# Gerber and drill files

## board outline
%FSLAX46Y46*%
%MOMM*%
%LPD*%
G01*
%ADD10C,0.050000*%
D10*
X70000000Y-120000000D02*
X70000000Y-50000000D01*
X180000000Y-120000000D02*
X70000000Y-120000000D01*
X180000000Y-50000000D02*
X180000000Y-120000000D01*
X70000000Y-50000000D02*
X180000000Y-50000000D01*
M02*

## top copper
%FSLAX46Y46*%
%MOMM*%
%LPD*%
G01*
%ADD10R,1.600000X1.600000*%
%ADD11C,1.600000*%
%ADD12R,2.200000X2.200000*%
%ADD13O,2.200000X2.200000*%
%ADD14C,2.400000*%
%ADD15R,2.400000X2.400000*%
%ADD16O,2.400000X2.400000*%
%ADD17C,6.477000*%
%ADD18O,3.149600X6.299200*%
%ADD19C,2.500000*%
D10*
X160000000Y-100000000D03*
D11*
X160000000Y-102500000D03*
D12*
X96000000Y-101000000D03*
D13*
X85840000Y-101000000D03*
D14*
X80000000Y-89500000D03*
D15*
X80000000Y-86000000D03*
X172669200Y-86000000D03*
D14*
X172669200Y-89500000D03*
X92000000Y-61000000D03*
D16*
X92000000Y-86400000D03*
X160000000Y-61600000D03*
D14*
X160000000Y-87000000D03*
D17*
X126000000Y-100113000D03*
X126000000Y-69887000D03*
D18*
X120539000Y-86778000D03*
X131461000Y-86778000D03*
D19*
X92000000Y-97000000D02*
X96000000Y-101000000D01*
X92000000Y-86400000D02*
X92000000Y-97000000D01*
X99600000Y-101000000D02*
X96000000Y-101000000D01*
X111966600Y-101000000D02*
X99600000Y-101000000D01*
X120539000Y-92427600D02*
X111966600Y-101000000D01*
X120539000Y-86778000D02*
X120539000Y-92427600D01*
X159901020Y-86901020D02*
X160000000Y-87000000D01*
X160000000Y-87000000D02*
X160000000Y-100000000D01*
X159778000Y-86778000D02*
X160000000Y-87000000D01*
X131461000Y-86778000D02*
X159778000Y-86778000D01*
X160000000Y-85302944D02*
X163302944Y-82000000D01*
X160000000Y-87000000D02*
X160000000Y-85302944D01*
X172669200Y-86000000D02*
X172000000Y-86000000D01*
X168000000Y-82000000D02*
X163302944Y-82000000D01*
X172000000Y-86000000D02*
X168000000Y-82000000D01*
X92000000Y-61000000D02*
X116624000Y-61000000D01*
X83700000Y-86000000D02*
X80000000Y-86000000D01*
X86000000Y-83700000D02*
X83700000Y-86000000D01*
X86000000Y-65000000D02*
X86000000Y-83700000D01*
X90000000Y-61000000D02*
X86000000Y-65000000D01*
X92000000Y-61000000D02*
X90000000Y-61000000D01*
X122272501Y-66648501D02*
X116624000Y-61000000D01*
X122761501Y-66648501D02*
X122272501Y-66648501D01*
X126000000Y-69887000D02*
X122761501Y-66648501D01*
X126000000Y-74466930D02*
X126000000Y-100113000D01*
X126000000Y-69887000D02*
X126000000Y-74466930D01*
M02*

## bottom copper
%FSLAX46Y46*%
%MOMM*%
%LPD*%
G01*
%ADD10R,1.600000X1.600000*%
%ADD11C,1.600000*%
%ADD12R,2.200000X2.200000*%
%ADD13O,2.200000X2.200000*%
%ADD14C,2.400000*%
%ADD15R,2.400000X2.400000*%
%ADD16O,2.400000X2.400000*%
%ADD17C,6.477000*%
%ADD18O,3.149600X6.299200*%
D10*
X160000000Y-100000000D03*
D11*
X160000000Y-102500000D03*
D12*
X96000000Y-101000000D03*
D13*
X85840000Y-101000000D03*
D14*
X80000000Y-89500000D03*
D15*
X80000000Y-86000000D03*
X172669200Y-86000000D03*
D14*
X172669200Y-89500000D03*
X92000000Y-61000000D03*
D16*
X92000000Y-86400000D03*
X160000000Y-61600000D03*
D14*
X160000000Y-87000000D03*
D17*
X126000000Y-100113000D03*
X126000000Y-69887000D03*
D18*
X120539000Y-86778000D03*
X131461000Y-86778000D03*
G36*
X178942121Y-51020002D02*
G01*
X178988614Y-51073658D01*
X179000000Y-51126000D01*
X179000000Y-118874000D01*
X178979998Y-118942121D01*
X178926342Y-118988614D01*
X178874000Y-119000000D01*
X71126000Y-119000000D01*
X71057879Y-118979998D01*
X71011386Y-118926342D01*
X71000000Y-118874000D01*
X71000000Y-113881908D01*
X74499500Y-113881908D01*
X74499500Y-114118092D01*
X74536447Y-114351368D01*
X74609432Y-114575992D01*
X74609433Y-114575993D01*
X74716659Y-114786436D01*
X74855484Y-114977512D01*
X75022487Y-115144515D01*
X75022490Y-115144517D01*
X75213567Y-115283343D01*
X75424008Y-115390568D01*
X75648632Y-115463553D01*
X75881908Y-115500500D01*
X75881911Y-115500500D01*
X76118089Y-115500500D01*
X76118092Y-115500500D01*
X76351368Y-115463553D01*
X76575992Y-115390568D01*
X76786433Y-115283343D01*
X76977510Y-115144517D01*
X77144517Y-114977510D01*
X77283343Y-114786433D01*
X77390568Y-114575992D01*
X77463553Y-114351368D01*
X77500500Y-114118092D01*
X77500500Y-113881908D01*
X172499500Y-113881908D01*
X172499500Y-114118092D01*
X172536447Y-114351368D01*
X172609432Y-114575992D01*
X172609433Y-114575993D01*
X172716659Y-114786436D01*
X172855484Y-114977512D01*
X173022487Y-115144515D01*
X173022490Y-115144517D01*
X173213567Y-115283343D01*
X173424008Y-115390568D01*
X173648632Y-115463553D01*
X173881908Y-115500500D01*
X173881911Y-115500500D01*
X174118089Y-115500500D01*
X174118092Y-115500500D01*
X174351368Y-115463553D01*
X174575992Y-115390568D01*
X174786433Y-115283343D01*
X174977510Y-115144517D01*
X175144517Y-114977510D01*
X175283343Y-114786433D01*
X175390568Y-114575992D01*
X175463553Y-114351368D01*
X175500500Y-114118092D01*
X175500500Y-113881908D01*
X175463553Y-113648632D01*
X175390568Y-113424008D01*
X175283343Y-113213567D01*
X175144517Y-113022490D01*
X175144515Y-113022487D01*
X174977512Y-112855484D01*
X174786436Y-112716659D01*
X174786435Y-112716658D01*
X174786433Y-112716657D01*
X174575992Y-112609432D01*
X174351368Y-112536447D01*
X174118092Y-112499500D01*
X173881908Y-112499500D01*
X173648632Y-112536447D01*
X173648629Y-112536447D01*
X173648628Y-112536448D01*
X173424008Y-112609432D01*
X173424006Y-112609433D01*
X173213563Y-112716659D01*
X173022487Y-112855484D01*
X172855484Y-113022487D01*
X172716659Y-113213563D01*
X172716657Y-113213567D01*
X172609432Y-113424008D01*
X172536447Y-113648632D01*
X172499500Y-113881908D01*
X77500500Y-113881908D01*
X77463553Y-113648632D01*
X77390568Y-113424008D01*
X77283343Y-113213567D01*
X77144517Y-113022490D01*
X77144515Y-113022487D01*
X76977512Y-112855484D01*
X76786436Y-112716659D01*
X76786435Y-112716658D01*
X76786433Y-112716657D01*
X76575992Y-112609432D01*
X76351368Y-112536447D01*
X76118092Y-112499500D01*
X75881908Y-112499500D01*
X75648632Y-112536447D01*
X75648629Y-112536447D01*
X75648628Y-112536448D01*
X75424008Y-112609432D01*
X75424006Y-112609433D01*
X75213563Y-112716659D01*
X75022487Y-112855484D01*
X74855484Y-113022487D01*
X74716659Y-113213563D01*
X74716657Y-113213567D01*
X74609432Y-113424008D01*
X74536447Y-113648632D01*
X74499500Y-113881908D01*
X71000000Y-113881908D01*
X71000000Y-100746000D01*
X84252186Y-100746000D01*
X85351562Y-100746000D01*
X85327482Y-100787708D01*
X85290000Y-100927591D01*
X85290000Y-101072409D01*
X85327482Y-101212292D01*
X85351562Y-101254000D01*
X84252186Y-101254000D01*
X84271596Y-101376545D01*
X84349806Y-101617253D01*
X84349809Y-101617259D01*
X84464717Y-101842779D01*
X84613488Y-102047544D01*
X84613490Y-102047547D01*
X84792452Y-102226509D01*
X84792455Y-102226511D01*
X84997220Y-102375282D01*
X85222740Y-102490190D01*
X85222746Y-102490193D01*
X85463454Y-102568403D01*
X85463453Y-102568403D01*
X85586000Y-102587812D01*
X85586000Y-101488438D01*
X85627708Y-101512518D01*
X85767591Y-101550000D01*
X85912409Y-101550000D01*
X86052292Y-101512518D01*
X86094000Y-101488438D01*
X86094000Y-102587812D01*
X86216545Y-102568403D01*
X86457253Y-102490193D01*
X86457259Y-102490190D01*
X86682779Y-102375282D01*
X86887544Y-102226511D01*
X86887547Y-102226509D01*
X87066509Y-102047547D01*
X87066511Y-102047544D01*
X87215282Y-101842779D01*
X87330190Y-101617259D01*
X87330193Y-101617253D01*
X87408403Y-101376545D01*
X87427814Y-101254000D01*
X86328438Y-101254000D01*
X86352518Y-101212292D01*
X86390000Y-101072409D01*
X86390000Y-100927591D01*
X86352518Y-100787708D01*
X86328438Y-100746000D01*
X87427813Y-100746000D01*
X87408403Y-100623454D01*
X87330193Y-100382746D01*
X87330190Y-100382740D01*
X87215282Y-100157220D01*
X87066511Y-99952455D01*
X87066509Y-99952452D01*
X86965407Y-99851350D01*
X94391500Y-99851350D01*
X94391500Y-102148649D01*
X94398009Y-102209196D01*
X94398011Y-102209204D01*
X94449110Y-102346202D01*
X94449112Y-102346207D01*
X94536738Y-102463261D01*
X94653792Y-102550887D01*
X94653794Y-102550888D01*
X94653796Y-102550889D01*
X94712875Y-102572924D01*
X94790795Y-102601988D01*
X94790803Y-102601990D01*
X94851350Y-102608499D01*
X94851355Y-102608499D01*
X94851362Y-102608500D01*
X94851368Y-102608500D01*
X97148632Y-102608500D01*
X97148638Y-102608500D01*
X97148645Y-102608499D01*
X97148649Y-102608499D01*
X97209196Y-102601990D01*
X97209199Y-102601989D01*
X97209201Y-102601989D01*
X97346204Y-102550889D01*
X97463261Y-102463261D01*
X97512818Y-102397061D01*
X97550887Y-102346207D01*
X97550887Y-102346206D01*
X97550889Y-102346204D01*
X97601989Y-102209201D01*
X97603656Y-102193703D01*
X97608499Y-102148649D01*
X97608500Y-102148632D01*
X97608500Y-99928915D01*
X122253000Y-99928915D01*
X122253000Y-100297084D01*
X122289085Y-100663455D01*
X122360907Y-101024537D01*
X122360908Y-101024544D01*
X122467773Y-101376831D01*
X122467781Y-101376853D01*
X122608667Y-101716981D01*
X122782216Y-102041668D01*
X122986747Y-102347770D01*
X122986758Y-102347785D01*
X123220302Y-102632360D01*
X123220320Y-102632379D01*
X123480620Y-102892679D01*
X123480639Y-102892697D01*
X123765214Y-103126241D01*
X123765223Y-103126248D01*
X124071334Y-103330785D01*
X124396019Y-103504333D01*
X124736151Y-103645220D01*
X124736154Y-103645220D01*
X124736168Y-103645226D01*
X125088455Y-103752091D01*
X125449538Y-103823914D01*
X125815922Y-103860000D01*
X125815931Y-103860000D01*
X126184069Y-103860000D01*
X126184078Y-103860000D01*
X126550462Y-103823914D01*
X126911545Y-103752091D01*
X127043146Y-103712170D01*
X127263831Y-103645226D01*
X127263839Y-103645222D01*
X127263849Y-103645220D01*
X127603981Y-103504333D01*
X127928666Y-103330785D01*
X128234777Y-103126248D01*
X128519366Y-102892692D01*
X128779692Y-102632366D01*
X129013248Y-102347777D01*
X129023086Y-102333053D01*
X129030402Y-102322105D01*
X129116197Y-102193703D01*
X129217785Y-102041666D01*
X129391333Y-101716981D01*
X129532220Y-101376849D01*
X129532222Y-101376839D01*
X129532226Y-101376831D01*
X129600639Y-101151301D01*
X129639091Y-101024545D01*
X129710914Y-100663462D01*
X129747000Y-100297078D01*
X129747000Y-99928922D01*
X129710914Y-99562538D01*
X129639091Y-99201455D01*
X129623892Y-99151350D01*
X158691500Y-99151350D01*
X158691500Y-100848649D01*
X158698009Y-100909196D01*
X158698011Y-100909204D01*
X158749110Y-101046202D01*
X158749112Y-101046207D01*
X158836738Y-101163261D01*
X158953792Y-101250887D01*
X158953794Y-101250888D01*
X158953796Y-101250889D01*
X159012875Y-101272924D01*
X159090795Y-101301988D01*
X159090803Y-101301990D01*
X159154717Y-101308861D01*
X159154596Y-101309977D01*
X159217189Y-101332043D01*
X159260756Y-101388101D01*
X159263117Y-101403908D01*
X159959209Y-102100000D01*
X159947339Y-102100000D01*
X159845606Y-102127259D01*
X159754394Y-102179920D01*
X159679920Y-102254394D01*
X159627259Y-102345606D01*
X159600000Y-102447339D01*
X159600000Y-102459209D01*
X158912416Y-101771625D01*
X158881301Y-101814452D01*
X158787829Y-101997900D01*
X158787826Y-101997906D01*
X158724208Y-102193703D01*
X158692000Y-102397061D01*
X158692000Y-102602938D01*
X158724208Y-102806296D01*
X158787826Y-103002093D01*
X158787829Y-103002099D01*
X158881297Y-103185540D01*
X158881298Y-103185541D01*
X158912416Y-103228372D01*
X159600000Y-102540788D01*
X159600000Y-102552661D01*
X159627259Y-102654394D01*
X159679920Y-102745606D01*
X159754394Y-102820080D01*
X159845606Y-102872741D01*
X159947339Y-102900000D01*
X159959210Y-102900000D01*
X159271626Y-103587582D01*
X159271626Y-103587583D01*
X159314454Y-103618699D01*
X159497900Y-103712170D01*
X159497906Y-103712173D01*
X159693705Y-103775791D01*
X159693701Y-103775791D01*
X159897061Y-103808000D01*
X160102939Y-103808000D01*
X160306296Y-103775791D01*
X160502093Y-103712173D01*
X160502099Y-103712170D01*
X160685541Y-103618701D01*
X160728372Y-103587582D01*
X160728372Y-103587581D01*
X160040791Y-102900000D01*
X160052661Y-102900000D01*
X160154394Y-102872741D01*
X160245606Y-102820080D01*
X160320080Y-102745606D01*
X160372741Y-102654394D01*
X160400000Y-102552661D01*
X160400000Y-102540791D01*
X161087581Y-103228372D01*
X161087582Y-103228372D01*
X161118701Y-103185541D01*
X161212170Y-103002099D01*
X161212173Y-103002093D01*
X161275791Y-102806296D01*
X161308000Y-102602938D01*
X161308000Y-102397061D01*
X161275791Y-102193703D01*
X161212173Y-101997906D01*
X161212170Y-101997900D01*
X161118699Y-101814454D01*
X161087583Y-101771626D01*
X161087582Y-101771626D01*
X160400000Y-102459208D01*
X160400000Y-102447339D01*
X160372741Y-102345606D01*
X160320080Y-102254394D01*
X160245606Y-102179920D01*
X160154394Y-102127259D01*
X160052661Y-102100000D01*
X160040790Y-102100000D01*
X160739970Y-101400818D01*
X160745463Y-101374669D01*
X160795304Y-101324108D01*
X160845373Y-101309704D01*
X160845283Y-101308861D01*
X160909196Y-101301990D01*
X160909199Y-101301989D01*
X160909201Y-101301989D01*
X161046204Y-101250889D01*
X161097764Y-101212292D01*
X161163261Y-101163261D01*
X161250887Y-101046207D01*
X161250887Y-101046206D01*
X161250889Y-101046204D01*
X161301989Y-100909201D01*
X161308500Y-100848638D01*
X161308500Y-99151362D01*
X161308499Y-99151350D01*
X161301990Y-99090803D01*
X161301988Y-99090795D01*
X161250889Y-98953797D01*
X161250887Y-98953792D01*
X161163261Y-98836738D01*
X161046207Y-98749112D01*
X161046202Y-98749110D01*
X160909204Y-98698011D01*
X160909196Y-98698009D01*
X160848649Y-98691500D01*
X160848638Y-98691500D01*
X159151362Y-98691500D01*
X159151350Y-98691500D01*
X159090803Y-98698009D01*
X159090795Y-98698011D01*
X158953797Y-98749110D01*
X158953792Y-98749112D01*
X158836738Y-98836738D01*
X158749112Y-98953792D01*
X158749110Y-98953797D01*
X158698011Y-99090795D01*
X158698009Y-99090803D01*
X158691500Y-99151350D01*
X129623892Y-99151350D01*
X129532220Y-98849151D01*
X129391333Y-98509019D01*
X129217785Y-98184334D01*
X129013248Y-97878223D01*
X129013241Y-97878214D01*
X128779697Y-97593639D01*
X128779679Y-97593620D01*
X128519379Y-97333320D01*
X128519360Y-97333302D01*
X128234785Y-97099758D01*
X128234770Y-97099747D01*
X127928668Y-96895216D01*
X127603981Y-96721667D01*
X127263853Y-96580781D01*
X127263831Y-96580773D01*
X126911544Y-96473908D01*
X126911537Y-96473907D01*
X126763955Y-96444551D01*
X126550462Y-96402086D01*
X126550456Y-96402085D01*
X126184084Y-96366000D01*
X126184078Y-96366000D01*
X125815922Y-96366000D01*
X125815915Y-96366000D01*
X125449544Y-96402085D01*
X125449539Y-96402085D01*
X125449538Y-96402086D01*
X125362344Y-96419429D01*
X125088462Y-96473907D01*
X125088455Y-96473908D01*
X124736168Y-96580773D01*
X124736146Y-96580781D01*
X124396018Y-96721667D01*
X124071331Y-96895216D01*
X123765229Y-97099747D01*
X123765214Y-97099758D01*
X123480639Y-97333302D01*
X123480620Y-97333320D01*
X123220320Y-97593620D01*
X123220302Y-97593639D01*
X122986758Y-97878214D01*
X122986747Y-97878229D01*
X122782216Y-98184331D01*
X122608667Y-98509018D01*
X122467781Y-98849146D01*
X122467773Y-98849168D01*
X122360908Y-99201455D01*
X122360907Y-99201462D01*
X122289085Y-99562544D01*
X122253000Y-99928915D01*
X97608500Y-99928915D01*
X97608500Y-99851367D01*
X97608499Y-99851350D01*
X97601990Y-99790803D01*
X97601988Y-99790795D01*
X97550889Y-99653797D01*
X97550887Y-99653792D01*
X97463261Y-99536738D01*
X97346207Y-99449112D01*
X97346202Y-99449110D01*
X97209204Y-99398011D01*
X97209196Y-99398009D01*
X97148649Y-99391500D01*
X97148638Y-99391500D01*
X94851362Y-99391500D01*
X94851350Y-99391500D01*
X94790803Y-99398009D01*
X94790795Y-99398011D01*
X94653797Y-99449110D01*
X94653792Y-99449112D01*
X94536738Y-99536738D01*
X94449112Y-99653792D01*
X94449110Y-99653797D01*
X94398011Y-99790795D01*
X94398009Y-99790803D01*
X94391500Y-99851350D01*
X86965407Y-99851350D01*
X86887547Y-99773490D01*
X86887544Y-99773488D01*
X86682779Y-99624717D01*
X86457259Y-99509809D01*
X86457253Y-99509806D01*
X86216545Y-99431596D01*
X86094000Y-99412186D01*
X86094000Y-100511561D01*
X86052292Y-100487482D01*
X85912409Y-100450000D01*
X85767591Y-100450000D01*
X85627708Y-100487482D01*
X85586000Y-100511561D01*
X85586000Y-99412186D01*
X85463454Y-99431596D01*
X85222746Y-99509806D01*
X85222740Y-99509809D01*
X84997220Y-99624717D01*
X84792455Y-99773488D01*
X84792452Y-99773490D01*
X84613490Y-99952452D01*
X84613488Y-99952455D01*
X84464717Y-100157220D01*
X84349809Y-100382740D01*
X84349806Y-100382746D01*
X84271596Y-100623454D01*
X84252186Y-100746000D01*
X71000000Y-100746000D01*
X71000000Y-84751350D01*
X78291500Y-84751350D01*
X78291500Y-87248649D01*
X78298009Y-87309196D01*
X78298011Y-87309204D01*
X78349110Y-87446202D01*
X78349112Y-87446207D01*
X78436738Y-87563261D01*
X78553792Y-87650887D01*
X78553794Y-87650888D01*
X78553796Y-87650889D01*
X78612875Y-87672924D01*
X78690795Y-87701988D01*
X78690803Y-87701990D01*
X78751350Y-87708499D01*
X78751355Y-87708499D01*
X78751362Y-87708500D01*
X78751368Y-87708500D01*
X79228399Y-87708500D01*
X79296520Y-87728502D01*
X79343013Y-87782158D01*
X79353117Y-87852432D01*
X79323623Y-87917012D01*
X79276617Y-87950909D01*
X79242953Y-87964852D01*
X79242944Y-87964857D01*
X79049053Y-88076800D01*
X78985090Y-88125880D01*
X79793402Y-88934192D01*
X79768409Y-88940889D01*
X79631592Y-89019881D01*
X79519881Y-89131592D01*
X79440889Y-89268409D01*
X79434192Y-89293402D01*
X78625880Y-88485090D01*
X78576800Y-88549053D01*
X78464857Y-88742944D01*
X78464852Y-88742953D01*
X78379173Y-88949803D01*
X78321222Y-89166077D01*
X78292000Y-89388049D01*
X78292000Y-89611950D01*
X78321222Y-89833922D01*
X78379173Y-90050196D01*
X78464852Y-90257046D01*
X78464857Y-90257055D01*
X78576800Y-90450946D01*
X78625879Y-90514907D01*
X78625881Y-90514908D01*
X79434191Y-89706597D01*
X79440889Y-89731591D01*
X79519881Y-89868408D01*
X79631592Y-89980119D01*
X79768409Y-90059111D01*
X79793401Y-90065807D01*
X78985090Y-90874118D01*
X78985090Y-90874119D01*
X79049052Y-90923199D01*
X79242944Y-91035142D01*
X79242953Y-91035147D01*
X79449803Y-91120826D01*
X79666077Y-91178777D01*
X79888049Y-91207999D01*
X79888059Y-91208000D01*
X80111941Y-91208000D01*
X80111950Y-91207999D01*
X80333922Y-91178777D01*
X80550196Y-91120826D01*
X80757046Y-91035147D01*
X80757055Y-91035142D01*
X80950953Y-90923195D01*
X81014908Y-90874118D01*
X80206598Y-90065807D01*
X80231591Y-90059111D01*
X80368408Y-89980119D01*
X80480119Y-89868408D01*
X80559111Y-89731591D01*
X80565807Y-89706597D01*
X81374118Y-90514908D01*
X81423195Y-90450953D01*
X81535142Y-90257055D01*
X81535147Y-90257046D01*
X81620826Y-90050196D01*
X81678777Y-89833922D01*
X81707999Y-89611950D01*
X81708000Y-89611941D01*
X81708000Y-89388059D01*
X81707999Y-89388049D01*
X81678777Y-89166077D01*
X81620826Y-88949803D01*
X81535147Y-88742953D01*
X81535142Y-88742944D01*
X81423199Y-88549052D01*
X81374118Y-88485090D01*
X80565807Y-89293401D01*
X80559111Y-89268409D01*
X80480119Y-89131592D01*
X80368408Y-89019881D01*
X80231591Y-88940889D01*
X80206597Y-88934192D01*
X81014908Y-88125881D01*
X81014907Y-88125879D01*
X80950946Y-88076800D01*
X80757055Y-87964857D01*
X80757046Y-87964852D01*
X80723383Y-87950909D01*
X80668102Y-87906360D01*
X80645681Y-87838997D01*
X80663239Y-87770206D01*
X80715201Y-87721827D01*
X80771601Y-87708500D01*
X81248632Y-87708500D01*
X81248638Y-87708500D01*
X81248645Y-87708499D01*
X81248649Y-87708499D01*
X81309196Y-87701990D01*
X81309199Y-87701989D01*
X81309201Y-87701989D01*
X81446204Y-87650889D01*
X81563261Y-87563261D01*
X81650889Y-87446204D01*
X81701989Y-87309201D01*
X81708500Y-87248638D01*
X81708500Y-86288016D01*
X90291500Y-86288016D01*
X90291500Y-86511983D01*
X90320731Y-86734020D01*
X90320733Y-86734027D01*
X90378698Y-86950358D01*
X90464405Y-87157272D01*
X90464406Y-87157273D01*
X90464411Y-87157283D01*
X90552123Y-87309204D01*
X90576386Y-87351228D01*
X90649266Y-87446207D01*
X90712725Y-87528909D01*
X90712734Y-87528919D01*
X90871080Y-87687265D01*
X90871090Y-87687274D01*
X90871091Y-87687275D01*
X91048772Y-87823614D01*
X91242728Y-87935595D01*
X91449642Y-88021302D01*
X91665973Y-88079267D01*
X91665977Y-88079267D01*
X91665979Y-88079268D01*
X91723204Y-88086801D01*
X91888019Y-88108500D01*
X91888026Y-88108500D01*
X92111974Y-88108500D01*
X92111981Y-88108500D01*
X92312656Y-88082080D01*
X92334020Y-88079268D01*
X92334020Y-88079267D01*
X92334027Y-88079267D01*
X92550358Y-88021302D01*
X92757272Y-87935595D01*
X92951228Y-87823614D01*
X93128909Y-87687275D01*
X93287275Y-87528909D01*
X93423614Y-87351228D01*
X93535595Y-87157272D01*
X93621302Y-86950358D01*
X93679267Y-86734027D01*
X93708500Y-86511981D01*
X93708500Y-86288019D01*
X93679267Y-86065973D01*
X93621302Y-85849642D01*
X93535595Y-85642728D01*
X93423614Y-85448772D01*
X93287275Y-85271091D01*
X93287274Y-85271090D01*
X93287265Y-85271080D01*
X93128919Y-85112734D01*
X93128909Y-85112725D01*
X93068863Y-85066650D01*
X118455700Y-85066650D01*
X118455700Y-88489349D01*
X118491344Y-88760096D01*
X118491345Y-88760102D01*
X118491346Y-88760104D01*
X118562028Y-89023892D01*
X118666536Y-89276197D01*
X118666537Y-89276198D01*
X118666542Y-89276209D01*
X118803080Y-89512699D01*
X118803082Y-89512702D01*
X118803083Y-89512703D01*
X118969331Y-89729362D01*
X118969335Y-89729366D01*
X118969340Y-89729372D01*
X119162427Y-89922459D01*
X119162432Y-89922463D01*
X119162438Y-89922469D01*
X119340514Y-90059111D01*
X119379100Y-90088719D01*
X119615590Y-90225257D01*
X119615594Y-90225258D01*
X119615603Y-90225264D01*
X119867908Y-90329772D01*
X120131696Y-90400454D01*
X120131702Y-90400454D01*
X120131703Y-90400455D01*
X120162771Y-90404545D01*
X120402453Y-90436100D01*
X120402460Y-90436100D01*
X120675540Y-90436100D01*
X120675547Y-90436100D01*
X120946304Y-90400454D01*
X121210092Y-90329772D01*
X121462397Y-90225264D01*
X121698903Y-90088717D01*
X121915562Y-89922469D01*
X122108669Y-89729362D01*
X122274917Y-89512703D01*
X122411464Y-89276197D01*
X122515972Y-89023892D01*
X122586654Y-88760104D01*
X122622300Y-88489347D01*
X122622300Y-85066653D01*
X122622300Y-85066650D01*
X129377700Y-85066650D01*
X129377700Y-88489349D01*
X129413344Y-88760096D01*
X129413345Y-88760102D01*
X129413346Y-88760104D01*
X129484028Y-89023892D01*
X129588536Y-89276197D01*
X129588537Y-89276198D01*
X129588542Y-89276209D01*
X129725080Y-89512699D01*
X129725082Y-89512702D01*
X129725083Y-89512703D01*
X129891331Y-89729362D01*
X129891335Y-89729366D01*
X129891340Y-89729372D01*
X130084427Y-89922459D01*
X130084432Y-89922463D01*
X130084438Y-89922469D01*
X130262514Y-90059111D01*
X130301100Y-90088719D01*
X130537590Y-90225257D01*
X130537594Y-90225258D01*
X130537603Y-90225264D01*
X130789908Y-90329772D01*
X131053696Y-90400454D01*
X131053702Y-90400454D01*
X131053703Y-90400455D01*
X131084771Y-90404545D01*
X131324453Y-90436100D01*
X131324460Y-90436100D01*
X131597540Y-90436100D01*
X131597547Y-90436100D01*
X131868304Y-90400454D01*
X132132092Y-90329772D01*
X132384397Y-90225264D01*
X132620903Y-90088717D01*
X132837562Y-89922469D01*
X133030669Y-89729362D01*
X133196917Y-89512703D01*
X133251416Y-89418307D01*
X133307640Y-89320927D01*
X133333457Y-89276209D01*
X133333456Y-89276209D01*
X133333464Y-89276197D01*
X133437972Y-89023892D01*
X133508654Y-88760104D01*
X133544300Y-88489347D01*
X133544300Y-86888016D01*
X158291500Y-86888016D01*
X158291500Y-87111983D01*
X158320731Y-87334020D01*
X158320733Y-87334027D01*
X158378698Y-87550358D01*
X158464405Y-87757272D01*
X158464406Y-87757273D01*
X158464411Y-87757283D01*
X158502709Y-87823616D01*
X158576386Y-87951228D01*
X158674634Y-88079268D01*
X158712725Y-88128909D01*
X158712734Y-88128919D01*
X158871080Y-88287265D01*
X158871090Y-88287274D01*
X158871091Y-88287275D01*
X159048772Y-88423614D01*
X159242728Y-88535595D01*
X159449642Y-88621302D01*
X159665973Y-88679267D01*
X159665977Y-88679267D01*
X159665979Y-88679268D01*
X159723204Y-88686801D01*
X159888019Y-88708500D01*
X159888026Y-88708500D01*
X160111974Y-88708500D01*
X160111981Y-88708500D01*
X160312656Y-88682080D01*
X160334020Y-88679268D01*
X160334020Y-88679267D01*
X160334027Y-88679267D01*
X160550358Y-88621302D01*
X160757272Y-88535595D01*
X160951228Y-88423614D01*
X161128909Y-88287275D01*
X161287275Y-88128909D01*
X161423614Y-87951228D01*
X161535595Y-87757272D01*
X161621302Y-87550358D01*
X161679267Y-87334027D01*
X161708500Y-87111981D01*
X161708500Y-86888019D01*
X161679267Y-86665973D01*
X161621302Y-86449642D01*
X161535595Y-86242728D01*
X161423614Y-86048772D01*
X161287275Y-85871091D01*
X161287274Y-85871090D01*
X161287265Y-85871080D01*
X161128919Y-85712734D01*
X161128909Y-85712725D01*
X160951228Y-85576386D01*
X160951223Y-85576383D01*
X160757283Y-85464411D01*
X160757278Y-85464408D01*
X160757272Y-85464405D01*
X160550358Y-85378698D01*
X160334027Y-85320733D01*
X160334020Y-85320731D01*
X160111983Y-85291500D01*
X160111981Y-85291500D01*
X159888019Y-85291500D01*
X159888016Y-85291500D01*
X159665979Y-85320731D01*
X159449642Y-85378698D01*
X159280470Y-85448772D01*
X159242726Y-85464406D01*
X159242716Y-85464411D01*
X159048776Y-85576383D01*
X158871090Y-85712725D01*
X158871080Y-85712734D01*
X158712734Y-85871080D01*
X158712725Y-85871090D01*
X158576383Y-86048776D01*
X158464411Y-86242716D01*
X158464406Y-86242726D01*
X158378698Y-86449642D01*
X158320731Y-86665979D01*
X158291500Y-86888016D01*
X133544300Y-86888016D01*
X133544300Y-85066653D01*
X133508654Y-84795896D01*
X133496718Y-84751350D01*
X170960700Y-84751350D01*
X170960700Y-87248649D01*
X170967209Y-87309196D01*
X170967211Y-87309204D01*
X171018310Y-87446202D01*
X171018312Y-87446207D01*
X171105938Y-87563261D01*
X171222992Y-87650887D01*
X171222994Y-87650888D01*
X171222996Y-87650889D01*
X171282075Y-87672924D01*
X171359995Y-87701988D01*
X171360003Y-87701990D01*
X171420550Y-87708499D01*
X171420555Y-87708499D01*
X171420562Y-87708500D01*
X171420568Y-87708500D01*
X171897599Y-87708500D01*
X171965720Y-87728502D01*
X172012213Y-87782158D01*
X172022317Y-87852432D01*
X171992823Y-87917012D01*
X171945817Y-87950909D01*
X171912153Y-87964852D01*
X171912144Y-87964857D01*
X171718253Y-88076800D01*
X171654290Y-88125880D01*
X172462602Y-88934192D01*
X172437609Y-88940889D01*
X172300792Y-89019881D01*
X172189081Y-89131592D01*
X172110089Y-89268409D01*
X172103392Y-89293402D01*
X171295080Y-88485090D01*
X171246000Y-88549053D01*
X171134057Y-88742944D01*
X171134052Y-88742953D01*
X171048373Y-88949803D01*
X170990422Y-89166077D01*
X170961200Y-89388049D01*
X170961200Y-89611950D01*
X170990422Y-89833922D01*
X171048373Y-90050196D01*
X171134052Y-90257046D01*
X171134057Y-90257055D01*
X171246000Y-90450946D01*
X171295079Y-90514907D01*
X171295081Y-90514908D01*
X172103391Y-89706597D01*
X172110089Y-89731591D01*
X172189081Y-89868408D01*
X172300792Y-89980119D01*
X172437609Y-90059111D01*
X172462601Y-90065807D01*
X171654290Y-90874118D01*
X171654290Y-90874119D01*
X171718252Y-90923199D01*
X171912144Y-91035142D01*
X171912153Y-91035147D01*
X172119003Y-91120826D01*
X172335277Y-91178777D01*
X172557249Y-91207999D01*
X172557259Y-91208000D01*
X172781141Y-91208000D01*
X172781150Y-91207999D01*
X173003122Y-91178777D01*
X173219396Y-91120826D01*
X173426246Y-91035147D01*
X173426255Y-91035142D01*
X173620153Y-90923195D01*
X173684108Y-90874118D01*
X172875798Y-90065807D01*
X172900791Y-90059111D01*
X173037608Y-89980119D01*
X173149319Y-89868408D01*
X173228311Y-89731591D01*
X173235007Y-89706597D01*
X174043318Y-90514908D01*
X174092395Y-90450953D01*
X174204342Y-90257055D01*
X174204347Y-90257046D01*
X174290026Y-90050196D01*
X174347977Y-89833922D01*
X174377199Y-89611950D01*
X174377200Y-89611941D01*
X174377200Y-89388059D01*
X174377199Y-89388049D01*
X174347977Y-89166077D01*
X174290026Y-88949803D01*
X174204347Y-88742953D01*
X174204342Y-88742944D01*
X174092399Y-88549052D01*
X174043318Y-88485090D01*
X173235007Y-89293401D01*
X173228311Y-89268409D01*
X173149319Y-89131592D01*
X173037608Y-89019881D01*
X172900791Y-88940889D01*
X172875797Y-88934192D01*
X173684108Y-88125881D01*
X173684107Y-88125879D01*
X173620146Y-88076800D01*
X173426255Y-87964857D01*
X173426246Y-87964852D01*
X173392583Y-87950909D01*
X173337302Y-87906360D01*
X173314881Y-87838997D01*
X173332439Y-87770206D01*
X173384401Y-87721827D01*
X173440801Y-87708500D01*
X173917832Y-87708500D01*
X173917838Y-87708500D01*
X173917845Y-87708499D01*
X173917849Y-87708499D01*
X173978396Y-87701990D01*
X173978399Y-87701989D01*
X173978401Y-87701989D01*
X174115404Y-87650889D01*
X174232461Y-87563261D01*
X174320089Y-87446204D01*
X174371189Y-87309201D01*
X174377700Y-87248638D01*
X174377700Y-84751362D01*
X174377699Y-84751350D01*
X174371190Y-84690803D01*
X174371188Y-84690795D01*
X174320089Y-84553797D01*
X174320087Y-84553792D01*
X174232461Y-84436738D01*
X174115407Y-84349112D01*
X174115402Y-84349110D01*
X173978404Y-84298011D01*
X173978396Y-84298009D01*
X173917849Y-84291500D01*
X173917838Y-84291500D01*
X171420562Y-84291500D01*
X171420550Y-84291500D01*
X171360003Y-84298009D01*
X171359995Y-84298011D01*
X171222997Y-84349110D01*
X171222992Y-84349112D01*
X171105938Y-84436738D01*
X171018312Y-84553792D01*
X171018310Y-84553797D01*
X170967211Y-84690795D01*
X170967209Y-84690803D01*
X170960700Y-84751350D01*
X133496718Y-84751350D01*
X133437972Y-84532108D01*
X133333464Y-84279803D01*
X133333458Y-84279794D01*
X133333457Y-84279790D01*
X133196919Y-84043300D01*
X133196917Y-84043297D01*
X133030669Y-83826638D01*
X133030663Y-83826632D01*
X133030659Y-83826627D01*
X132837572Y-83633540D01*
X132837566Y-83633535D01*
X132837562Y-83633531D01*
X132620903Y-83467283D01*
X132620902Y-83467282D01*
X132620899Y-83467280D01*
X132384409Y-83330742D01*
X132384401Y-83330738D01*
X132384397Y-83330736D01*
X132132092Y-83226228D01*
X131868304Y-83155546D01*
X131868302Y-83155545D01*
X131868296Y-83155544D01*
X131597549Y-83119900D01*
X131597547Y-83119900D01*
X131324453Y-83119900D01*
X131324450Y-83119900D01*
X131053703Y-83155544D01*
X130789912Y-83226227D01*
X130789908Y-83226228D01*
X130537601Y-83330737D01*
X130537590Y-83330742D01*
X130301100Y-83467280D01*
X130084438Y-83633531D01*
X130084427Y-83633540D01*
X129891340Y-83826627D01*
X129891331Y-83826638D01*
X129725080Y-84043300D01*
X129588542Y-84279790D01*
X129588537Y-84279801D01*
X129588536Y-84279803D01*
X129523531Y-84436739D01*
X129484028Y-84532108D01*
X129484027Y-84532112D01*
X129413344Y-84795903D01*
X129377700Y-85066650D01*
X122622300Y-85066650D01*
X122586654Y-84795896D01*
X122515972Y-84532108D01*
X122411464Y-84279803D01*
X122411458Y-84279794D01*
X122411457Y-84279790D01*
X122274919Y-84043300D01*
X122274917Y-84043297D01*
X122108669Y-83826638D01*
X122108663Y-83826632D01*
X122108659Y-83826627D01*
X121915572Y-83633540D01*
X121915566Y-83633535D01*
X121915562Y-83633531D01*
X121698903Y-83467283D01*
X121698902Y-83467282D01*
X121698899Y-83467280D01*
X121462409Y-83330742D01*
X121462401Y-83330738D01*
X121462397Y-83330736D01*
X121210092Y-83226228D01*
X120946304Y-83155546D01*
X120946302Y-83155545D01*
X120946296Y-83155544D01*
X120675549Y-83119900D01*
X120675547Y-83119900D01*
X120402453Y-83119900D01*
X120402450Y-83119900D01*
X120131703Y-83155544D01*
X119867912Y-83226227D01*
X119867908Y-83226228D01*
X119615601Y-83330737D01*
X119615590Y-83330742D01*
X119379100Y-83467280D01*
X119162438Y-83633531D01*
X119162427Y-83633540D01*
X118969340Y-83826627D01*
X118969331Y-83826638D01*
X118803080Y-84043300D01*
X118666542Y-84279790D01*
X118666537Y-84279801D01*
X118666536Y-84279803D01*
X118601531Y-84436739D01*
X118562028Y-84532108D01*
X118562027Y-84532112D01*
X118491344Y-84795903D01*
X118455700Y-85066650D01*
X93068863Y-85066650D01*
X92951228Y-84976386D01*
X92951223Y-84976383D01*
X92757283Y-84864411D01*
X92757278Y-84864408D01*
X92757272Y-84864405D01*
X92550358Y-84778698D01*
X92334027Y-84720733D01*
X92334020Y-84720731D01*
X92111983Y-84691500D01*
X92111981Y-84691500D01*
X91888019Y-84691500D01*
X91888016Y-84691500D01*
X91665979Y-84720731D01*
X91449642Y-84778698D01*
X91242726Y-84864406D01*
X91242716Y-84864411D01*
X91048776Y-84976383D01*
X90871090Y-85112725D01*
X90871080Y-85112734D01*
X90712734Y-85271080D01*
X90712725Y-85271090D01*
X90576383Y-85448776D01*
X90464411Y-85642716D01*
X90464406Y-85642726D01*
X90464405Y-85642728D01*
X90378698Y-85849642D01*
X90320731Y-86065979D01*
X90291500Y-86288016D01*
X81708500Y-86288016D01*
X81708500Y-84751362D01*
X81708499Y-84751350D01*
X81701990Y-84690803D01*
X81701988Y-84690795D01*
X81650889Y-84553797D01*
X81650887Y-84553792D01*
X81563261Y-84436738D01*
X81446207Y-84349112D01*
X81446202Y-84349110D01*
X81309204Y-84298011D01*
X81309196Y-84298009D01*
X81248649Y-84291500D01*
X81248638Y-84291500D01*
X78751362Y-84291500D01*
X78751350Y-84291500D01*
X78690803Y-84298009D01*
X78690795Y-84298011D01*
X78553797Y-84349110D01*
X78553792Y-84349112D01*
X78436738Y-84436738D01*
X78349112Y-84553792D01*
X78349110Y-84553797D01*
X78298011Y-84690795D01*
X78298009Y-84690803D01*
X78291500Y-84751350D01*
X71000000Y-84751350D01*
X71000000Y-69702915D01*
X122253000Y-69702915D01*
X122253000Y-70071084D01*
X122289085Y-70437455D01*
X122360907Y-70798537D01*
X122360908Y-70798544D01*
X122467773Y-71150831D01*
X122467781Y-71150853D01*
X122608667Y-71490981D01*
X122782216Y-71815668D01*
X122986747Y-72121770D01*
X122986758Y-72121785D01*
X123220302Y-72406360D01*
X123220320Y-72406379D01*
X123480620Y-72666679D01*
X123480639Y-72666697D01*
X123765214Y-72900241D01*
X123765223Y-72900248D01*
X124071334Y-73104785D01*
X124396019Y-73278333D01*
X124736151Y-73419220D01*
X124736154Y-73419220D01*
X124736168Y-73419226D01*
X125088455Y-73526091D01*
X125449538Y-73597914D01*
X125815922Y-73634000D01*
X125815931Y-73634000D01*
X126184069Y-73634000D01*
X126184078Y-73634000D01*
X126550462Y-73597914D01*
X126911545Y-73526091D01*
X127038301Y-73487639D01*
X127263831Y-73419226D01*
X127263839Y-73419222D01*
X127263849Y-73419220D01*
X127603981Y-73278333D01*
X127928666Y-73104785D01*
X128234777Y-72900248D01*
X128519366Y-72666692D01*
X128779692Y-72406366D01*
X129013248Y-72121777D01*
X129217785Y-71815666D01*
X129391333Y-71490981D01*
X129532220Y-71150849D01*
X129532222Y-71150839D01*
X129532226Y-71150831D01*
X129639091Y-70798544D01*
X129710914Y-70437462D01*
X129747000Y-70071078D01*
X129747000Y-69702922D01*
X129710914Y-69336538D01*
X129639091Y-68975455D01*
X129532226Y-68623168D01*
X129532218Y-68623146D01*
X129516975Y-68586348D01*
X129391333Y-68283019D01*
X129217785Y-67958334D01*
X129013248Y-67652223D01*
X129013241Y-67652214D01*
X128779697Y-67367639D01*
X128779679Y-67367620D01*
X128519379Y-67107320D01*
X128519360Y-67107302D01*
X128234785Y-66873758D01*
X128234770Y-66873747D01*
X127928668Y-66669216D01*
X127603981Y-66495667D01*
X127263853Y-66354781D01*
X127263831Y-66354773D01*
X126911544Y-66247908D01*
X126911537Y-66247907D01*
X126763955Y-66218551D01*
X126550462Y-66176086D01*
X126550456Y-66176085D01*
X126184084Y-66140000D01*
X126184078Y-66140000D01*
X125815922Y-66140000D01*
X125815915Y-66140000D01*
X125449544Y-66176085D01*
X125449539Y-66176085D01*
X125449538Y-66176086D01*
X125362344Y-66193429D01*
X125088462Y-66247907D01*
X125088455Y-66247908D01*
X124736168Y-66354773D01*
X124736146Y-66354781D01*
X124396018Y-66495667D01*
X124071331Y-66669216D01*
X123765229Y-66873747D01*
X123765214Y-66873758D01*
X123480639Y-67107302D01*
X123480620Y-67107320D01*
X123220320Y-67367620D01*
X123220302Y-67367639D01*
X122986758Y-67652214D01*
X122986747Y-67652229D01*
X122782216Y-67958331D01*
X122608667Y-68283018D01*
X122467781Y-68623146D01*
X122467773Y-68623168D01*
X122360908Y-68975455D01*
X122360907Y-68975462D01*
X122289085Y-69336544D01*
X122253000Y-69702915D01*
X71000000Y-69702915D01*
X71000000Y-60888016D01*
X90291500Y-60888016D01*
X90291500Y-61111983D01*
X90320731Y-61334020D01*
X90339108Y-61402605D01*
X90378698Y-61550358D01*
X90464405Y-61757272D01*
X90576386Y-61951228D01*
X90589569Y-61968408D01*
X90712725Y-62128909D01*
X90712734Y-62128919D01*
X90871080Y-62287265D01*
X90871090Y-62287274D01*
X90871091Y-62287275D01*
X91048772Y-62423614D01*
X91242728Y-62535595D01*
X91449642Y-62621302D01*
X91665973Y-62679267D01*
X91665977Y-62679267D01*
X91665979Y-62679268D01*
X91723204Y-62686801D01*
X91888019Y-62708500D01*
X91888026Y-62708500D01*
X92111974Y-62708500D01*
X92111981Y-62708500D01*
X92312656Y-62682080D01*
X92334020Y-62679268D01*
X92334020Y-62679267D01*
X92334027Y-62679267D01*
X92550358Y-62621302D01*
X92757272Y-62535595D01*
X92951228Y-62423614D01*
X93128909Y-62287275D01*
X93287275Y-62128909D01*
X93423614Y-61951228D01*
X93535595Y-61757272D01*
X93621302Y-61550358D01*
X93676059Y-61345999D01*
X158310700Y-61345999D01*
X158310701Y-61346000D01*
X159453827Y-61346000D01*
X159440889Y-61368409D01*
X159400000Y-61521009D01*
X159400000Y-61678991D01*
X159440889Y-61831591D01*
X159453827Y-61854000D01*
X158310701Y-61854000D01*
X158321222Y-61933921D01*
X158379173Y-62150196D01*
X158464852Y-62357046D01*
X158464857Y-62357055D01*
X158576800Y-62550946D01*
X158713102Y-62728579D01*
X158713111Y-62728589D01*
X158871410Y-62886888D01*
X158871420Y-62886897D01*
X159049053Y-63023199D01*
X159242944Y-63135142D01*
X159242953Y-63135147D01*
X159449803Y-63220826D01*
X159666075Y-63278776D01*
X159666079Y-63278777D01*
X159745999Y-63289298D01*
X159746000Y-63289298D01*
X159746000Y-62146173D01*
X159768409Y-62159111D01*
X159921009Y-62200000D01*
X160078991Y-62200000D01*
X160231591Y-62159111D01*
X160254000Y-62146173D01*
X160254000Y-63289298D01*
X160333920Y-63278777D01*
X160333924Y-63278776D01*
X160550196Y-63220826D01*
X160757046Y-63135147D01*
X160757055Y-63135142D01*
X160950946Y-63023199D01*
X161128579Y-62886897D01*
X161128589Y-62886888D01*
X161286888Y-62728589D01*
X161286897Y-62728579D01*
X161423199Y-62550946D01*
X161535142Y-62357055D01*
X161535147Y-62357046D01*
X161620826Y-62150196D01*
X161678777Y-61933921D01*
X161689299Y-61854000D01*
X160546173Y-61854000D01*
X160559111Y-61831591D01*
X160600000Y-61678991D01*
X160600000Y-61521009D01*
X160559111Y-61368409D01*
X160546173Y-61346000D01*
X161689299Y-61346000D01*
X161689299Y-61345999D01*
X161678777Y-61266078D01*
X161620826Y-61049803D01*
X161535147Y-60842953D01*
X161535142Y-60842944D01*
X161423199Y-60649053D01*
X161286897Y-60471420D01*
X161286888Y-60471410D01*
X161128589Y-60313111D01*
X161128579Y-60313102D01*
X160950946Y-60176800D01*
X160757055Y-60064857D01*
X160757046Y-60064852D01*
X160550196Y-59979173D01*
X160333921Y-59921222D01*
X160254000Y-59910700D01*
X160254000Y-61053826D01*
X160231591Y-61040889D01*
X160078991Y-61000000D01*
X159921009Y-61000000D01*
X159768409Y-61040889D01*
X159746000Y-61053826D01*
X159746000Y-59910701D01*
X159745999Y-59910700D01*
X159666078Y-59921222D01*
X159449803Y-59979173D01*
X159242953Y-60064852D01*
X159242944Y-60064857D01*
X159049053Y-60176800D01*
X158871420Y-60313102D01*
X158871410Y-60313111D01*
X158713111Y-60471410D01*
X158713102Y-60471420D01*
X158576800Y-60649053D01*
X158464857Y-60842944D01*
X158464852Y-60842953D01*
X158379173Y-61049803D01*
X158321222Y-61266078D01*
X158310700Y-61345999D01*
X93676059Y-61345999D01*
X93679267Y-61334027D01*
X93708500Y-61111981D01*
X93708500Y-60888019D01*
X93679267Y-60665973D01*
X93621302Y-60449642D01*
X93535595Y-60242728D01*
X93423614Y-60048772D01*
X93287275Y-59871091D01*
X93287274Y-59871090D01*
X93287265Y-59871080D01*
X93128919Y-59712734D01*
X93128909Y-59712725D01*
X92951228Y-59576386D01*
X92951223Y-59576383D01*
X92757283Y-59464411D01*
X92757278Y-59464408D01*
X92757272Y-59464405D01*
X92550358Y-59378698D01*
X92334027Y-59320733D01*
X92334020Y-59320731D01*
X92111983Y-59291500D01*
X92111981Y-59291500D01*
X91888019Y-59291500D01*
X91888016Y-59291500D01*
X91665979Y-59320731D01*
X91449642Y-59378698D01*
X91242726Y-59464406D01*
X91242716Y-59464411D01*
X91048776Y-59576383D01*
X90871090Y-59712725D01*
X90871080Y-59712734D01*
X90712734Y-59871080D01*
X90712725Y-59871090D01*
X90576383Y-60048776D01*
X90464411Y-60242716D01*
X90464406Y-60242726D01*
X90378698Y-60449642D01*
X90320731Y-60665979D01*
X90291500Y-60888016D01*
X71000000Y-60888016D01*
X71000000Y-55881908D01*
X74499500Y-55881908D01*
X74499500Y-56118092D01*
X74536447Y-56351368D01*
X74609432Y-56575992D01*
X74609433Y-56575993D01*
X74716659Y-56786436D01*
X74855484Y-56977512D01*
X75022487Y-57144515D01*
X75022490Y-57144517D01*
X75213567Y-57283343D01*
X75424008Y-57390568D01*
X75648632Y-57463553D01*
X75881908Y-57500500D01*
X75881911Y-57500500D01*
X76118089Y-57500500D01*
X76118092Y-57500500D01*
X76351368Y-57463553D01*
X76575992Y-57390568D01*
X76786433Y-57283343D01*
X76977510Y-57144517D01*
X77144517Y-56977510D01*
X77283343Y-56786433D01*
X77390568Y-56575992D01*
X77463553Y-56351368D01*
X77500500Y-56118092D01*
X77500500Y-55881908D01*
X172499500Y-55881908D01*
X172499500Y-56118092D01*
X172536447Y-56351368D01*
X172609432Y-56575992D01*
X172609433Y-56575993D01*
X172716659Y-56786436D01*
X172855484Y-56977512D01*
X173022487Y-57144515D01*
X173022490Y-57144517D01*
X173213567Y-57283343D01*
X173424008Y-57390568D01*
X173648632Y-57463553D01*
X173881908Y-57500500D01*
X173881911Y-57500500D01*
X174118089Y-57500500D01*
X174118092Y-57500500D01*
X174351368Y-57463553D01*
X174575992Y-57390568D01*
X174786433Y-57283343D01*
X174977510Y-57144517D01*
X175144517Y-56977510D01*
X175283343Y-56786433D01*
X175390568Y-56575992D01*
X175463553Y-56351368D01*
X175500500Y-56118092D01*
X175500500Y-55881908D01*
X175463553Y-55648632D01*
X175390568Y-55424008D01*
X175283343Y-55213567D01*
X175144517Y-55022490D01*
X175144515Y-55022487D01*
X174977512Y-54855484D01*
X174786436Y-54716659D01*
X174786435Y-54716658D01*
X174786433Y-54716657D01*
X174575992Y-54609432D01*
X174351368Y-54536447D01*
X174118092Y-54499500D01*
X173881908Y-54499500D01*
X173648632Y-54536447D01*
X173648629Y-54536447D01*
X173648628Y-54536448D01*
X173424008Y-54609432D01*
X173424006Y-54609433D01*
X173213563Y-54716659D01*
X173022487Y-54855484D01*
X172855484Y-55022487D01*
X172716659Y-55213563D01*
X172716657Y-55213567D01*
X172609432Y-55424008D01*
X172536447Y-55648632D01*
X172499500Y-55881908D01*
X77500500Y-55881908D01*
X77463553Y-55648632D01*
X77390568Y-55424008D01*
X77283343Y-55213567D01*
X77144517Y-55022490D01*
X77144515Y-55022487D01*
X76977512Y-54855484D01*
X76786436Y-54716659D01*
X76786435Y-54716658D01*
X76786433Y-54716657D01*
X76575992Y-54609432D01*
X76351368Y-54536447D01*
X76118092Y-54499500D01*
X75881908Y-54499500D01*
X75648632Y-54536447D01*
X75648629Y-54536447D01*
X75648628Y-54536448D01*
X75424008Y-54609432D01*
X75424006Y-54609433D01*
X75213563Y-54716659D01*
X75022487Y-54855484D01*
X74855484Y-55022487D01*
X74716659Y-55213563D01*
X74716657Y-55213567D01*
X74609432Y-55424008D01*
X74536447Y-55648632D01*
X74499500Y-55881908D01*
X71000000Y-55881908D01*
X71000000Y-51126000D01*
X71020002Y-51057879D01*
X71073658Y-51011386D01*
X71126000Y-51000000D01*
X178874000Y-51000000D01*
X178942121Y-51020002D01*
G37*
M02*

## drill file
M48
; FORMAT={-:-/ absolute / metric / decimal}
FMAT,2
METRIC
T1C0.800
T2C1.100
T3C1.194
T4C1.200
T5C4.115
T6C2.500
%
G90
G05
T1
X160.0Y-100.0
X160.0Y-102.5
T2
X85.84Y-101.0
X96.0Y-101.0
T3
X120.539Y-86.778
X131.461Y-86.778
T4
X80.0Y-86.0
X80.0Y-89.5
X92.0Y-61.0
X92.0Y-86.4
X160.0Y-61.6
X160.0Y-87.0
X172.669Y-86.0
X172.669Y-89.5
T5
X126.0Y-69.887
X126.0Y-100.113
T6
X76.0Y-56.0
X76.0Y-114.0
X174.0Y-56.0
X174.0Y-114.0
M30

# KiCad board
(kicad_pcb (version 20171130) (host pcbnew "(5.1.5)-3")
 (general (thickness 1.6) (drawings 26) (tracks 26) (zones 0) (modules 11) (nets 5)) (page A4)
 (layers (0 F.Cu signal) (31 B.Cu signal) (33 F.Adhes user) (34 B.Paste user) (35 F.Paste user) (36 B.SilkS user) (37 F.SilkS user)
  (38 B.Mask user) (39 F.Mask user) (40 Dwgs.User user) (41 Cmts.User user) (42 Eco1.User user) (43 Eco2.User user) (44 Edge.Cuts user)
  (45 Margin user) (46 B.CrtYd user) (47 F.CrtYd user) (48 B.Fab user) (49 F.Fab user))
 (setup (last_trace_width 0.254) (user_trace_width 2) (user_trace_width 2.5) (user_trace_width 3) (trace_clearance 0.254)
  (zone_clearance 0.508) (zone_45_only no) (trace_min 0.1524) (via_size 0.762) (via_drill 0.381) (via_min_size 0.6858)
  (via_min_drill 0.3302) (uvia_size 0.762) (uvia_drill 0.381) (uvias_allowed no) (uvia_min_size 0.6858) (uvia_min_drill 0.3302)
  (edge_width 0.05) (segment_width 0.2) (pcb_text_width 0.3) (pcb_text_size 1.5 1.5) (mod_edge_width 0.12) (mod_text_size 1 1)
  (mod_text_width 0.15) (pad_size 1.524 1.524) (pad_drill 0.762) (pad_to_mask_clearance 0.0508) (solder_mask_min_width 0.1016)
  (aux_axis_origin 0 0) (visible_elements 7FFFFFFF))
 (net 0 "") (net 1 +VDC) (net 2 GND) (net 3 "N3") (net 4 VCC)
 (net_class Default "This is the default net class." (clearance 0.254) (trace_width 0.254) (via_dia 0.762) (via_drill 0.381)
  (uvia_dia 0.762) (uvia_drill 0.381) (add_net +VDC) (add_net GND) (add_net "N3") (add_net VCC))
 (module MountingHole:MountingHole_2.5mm (layer F.Cu) (at 76 56)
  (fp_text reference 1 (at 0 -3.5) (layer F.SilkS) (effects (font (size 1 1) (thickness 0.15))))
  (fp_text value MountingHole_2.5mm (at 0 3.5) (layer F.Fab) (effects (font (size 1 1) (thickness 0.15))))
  (pad 1 np_thru_hole circle (at 0 0) (size 2.5 2.5) (drill 2.5) (layers *.Cu *.Mask)))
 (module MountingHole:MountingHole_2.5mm (layer F.Cu) (at 76 114)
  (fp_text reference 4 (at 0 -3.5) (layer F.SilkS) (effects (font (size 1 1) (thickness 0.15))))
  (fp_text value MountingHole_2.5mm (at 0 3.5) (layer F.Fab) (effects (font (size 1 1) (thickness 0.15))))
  (pad 1 np_thru_hole circle (at 0 0) (size 2.5 2.5) (drill 2.5) (layers *.Cu *.Mask)))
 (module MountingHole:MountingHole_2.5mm (layer F.Cu) (at 174 114)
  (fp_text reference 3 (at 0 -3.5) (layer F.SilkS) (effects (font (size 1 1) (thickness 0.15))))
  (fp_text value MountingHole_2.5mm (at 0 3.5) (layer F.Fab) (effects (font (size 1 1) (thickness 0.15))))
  (pad 1 np_thru_hole circle (at 0 0) (size 2.5 2.5) (drill 2.5) (layers *.Cu *.Mask)))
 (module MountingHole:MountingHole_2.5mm (layer F.Cu) (at 174 56)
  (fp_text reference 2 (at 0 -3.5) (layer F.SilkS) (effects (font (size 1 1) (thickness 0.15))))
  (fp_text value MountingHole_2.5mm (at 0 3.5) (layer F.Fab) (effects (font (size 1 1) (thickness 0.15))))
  (pad 1 np_thru_hole circle (at 0 0) (size 2.5 2.5) (drill 2.5) (layers *.Cu *.Mask)))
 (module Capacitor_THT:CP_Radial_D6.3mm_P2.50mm (layer F.Cu) (at 160 100 270)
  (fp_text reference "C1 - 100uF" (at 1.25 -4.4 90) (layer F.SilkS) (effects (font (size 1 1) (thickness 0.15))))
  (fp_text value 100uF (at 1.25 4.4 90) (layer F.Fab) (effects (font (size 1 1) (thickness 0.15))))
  (pad 1 thru_hole rect (at 0 0 270) (size 1.6 1.6) (drill 0.8) (layers *.Cu *.Mask) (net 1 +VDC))
  (pad 2 thru_hole circle (at 2.5 0 270) (size 1.6 1.6) (drill 0.8) (layers *.Cu *.Mask) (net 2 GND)))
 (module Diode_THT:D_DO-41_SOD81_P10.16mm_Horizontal (layer F.Cu) (at 96 101 180)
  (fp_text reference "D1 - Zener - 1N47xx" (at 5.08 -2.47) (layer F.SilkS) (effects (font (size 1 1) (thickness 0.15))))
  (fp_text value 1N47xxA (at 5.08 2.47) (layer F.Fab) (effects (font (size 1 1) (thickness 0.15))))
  (pad 1 thru_hole rect (at 0 0 180) (size 2.2 2.2) (drill 1.1) (layers *.Cu *.Mask) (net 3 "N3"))
  (pad 2 thru_hole oval (at 10.16 0 180) (size 2.2 2.2) (drill 1.1) (layers *.Cu *.Mask) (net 2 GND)))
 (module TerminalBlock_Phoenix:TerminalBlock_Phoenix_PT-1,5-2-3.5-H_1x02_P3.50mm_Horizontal (layer F.Cu) (at 80 86 270)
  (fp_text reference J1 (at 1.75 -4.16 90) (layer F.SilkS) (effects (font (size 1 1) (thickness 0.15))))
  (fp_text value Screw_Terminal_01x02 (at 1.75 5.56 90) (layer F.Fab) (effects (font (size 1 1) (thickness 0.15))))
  (pad 2 thru_hole circle (at 3.5 0 270) (size 2.4 2.4) (drill 1.2) (layers *.Cu *.Mask) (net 2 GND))
  (pad 1 thru_hole rect (at 0 0 270) (size 2.4 2.4) (drill 1.2) (layers *.Cu *.Mask) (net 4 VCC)))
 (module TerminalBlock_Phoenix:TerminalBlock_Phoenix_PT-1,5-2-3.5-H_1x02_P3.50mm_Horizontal (layer F.Cu) (at 172.6692 86 270)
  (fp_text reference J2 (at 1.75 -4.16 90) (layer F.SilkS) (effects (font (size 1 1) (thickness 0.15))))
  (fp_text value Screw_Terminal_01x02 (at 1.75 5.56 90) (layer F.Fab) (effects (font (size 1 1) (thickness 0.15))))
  (pad 1 thru_hole rect (at 0 0 270) (size 2.4 2.4) (drill 1.2) (layers *.Cu *.Mask) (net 1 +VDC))
  (pad 2 thru_hole circle (at 3.5 0 270) (size 2.4 2.4) (drill 1.2) (layers *.Cu *.Mask) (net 2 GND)))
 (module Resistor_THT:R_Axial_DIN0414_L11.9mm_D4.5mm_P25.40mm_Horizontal (layer F.Cu) (at 92 61 270)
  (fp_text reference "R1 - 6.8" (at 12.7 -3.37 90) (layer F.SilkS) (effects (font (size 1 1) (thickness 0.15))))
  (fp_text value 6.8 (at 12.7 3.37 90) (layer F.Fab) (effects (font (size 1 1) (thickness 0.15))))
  (pad 1 thru_hole circle (at 0 0 270) (size 2.4 2.4) (drill 1.2) (layers *.Cu *.Mask) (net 4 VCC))
  (pad 2 thru_hole oval (at 25.4 0 270) (size 2.4 2.4) (drill 1.2) (layers *.Cu *.Mask) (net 3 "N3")))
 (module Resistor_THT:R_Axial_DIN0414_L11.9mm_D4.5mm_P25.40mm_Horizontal (layer F.Cu) (at 160 87 90)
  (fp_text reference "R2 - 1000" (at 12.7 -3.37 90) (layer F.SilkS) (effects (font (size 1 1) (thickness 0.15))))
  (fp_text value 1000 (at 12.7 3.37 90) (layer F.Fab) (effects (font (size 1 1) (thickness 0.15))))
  (pad 2 thru_hole oval (at 25.4 0 90) (size 2.4 2.4) (drill 1.2) (layers *.Cu *.Mask) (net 2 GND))
  (pad 1 thru_hole circle (at 0 0 90) (size 2.4 2.4) (drill 1.2) (layers *.Cu *.Mask) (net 1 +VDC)))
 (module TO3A (layer F.Cu) (at 126 85 90)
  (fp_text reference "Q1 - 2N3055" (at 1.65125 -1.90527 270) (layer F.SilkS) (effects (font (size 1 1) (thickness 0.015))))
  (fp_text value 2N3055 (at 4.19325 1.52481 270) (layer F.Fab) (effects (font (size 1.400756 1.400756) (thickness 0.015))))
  (pad C1 thru_hole circle (at -15.113 0 90) (size 6.477 6.477) (drill 4.1148) (layers *.Cu *.Mask) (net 4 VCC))
  (pad C thru_hole circle (at 15.113 0 90) (size 6.477 6.477) (drill 4.1148) (layers *.Cu *.Mask) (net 4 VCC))
  (pad B thru_hole oval (at -1.778 -5.461 90) (size 6.2992 3.1496) (drill 1.1938) (layers *.Cu *.Mask) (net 3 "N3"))
  (pad E thru_hole oval (at -1.778 5.461 90) (size 6.2992 3.1496) (drill 1.1938) (layers *.Cu *.Mask) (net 1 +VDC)))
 (gr_line (start 70 120) (end 70 50) (layer Edge.Cuts) (width 0.05))
 (gr_line (start 180 120) (end 70 120) (layer Edge.Cuts) (width 0.05))
 (gr_line (start 180 50) (end 180 120) (layer Edge.Cuts) (width 0.05))
 (gr_line (start 70 50) (end 180 50) (layer Edge.Cuts) (width 0.05))
 (segment (start 92 97) (end 96 101) (width 2.5) (layer F.Cu) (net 3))
 (segment (start 92 86.4) (end 92 97) (width 2.5) (layer F.Cu) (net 3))
 (segment (start 99.6 101) (end 96 101) (width 2.5) (layer F.Cu) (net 3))
 (segment (start 111.9666 101) (end 99.6 101) (width 2.5) (layer F.Cu) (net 3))
 (segment (start 120.539 92.4276) (end 111.9666 101) (width 2.5) (layer F.Cu) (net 3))
 (segment (start 120.539 86.778) (end 120.539 92.4276) (width 2.5) (layer F.Cu) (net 3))
 (segment (start 159.90102 86.90102) (end 160 87) (width 2.5) (layer F.Cu) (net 1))
 (segment (start 160 87) (end 160 100) (width 2.5) (layer F.Cu) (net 1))
 (segment (start 159.778 86.778) (end 160 87) (width 2.5) (layer F.Cu) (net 1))
 (segment (start 131.461 86.778) (end 159.778 86.778) (width 2.5) (layer F.Cu) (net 1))
 (segment (start 160 85.302944) (end 163.302944 82) (width 2.5) (layer F.Cu) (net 1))
 (segment (start 160 87) (end 160 85.302944) (width 2.5) (layer F.Cu) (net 1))
 (segment (start 172.6692 86) (end 172 86) (width 2.5) (layer F.Cu) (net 1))
 (segment (start 168 82) (end 163.302944 82) (width 2.5) (layer F.Cu) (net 1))
 (segment (start 172 86) (end 168 82) (width 2.5) (layer F.Cu) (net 1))
 (segment (start 92 61) (end 116.624 61) (width 2.5) (layer F.Cu) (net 4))
 (segment (start 83.7 86) (end 80 86) (width 2.5) (layer F.Cu) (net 4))
 (segment (start 86 83.7) (end 83.7 86) (width 2.5) (layer F.Cu) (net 4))
 (segment (start 86 65) (end 86 83.7) (width 2.5) (layer F.Cu) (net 4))
 (segment (start 90 61) (end 86 65) (width 2.5) (layer F.Cu) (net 4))
 (segment (start 92 61) (end 90 61) (width 2.5) (layer F.Cu) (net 4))
 (segment (start 122.272501 66.648501) (end 116.624 61) (width 2.5) (layer F.Cu) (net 4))
 (segment (start 122.761501 66.648501) (end 122.272501 66.648501) (width 2.5) (layer F.Cu) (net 4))
 (segment (start 126 69.887) (end 122.761501 66.648501) (width 2.5) (layer F.Cu) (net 4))
 (segment (start 126 74.46693) (end 126 100.113) (width 2.5) (layer F.Cu) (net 4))
 (segment (start 126 69.887) (end 126 74.46693) (width 2.5) (layer F.Cu) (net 4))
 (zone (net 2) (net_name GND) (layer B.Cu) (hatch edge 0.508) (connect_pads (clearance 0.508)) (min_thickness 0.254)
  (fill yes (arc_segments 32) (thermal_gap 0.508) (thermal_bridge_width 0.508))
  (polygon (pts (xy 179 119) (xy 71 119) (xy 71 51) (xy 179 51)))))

